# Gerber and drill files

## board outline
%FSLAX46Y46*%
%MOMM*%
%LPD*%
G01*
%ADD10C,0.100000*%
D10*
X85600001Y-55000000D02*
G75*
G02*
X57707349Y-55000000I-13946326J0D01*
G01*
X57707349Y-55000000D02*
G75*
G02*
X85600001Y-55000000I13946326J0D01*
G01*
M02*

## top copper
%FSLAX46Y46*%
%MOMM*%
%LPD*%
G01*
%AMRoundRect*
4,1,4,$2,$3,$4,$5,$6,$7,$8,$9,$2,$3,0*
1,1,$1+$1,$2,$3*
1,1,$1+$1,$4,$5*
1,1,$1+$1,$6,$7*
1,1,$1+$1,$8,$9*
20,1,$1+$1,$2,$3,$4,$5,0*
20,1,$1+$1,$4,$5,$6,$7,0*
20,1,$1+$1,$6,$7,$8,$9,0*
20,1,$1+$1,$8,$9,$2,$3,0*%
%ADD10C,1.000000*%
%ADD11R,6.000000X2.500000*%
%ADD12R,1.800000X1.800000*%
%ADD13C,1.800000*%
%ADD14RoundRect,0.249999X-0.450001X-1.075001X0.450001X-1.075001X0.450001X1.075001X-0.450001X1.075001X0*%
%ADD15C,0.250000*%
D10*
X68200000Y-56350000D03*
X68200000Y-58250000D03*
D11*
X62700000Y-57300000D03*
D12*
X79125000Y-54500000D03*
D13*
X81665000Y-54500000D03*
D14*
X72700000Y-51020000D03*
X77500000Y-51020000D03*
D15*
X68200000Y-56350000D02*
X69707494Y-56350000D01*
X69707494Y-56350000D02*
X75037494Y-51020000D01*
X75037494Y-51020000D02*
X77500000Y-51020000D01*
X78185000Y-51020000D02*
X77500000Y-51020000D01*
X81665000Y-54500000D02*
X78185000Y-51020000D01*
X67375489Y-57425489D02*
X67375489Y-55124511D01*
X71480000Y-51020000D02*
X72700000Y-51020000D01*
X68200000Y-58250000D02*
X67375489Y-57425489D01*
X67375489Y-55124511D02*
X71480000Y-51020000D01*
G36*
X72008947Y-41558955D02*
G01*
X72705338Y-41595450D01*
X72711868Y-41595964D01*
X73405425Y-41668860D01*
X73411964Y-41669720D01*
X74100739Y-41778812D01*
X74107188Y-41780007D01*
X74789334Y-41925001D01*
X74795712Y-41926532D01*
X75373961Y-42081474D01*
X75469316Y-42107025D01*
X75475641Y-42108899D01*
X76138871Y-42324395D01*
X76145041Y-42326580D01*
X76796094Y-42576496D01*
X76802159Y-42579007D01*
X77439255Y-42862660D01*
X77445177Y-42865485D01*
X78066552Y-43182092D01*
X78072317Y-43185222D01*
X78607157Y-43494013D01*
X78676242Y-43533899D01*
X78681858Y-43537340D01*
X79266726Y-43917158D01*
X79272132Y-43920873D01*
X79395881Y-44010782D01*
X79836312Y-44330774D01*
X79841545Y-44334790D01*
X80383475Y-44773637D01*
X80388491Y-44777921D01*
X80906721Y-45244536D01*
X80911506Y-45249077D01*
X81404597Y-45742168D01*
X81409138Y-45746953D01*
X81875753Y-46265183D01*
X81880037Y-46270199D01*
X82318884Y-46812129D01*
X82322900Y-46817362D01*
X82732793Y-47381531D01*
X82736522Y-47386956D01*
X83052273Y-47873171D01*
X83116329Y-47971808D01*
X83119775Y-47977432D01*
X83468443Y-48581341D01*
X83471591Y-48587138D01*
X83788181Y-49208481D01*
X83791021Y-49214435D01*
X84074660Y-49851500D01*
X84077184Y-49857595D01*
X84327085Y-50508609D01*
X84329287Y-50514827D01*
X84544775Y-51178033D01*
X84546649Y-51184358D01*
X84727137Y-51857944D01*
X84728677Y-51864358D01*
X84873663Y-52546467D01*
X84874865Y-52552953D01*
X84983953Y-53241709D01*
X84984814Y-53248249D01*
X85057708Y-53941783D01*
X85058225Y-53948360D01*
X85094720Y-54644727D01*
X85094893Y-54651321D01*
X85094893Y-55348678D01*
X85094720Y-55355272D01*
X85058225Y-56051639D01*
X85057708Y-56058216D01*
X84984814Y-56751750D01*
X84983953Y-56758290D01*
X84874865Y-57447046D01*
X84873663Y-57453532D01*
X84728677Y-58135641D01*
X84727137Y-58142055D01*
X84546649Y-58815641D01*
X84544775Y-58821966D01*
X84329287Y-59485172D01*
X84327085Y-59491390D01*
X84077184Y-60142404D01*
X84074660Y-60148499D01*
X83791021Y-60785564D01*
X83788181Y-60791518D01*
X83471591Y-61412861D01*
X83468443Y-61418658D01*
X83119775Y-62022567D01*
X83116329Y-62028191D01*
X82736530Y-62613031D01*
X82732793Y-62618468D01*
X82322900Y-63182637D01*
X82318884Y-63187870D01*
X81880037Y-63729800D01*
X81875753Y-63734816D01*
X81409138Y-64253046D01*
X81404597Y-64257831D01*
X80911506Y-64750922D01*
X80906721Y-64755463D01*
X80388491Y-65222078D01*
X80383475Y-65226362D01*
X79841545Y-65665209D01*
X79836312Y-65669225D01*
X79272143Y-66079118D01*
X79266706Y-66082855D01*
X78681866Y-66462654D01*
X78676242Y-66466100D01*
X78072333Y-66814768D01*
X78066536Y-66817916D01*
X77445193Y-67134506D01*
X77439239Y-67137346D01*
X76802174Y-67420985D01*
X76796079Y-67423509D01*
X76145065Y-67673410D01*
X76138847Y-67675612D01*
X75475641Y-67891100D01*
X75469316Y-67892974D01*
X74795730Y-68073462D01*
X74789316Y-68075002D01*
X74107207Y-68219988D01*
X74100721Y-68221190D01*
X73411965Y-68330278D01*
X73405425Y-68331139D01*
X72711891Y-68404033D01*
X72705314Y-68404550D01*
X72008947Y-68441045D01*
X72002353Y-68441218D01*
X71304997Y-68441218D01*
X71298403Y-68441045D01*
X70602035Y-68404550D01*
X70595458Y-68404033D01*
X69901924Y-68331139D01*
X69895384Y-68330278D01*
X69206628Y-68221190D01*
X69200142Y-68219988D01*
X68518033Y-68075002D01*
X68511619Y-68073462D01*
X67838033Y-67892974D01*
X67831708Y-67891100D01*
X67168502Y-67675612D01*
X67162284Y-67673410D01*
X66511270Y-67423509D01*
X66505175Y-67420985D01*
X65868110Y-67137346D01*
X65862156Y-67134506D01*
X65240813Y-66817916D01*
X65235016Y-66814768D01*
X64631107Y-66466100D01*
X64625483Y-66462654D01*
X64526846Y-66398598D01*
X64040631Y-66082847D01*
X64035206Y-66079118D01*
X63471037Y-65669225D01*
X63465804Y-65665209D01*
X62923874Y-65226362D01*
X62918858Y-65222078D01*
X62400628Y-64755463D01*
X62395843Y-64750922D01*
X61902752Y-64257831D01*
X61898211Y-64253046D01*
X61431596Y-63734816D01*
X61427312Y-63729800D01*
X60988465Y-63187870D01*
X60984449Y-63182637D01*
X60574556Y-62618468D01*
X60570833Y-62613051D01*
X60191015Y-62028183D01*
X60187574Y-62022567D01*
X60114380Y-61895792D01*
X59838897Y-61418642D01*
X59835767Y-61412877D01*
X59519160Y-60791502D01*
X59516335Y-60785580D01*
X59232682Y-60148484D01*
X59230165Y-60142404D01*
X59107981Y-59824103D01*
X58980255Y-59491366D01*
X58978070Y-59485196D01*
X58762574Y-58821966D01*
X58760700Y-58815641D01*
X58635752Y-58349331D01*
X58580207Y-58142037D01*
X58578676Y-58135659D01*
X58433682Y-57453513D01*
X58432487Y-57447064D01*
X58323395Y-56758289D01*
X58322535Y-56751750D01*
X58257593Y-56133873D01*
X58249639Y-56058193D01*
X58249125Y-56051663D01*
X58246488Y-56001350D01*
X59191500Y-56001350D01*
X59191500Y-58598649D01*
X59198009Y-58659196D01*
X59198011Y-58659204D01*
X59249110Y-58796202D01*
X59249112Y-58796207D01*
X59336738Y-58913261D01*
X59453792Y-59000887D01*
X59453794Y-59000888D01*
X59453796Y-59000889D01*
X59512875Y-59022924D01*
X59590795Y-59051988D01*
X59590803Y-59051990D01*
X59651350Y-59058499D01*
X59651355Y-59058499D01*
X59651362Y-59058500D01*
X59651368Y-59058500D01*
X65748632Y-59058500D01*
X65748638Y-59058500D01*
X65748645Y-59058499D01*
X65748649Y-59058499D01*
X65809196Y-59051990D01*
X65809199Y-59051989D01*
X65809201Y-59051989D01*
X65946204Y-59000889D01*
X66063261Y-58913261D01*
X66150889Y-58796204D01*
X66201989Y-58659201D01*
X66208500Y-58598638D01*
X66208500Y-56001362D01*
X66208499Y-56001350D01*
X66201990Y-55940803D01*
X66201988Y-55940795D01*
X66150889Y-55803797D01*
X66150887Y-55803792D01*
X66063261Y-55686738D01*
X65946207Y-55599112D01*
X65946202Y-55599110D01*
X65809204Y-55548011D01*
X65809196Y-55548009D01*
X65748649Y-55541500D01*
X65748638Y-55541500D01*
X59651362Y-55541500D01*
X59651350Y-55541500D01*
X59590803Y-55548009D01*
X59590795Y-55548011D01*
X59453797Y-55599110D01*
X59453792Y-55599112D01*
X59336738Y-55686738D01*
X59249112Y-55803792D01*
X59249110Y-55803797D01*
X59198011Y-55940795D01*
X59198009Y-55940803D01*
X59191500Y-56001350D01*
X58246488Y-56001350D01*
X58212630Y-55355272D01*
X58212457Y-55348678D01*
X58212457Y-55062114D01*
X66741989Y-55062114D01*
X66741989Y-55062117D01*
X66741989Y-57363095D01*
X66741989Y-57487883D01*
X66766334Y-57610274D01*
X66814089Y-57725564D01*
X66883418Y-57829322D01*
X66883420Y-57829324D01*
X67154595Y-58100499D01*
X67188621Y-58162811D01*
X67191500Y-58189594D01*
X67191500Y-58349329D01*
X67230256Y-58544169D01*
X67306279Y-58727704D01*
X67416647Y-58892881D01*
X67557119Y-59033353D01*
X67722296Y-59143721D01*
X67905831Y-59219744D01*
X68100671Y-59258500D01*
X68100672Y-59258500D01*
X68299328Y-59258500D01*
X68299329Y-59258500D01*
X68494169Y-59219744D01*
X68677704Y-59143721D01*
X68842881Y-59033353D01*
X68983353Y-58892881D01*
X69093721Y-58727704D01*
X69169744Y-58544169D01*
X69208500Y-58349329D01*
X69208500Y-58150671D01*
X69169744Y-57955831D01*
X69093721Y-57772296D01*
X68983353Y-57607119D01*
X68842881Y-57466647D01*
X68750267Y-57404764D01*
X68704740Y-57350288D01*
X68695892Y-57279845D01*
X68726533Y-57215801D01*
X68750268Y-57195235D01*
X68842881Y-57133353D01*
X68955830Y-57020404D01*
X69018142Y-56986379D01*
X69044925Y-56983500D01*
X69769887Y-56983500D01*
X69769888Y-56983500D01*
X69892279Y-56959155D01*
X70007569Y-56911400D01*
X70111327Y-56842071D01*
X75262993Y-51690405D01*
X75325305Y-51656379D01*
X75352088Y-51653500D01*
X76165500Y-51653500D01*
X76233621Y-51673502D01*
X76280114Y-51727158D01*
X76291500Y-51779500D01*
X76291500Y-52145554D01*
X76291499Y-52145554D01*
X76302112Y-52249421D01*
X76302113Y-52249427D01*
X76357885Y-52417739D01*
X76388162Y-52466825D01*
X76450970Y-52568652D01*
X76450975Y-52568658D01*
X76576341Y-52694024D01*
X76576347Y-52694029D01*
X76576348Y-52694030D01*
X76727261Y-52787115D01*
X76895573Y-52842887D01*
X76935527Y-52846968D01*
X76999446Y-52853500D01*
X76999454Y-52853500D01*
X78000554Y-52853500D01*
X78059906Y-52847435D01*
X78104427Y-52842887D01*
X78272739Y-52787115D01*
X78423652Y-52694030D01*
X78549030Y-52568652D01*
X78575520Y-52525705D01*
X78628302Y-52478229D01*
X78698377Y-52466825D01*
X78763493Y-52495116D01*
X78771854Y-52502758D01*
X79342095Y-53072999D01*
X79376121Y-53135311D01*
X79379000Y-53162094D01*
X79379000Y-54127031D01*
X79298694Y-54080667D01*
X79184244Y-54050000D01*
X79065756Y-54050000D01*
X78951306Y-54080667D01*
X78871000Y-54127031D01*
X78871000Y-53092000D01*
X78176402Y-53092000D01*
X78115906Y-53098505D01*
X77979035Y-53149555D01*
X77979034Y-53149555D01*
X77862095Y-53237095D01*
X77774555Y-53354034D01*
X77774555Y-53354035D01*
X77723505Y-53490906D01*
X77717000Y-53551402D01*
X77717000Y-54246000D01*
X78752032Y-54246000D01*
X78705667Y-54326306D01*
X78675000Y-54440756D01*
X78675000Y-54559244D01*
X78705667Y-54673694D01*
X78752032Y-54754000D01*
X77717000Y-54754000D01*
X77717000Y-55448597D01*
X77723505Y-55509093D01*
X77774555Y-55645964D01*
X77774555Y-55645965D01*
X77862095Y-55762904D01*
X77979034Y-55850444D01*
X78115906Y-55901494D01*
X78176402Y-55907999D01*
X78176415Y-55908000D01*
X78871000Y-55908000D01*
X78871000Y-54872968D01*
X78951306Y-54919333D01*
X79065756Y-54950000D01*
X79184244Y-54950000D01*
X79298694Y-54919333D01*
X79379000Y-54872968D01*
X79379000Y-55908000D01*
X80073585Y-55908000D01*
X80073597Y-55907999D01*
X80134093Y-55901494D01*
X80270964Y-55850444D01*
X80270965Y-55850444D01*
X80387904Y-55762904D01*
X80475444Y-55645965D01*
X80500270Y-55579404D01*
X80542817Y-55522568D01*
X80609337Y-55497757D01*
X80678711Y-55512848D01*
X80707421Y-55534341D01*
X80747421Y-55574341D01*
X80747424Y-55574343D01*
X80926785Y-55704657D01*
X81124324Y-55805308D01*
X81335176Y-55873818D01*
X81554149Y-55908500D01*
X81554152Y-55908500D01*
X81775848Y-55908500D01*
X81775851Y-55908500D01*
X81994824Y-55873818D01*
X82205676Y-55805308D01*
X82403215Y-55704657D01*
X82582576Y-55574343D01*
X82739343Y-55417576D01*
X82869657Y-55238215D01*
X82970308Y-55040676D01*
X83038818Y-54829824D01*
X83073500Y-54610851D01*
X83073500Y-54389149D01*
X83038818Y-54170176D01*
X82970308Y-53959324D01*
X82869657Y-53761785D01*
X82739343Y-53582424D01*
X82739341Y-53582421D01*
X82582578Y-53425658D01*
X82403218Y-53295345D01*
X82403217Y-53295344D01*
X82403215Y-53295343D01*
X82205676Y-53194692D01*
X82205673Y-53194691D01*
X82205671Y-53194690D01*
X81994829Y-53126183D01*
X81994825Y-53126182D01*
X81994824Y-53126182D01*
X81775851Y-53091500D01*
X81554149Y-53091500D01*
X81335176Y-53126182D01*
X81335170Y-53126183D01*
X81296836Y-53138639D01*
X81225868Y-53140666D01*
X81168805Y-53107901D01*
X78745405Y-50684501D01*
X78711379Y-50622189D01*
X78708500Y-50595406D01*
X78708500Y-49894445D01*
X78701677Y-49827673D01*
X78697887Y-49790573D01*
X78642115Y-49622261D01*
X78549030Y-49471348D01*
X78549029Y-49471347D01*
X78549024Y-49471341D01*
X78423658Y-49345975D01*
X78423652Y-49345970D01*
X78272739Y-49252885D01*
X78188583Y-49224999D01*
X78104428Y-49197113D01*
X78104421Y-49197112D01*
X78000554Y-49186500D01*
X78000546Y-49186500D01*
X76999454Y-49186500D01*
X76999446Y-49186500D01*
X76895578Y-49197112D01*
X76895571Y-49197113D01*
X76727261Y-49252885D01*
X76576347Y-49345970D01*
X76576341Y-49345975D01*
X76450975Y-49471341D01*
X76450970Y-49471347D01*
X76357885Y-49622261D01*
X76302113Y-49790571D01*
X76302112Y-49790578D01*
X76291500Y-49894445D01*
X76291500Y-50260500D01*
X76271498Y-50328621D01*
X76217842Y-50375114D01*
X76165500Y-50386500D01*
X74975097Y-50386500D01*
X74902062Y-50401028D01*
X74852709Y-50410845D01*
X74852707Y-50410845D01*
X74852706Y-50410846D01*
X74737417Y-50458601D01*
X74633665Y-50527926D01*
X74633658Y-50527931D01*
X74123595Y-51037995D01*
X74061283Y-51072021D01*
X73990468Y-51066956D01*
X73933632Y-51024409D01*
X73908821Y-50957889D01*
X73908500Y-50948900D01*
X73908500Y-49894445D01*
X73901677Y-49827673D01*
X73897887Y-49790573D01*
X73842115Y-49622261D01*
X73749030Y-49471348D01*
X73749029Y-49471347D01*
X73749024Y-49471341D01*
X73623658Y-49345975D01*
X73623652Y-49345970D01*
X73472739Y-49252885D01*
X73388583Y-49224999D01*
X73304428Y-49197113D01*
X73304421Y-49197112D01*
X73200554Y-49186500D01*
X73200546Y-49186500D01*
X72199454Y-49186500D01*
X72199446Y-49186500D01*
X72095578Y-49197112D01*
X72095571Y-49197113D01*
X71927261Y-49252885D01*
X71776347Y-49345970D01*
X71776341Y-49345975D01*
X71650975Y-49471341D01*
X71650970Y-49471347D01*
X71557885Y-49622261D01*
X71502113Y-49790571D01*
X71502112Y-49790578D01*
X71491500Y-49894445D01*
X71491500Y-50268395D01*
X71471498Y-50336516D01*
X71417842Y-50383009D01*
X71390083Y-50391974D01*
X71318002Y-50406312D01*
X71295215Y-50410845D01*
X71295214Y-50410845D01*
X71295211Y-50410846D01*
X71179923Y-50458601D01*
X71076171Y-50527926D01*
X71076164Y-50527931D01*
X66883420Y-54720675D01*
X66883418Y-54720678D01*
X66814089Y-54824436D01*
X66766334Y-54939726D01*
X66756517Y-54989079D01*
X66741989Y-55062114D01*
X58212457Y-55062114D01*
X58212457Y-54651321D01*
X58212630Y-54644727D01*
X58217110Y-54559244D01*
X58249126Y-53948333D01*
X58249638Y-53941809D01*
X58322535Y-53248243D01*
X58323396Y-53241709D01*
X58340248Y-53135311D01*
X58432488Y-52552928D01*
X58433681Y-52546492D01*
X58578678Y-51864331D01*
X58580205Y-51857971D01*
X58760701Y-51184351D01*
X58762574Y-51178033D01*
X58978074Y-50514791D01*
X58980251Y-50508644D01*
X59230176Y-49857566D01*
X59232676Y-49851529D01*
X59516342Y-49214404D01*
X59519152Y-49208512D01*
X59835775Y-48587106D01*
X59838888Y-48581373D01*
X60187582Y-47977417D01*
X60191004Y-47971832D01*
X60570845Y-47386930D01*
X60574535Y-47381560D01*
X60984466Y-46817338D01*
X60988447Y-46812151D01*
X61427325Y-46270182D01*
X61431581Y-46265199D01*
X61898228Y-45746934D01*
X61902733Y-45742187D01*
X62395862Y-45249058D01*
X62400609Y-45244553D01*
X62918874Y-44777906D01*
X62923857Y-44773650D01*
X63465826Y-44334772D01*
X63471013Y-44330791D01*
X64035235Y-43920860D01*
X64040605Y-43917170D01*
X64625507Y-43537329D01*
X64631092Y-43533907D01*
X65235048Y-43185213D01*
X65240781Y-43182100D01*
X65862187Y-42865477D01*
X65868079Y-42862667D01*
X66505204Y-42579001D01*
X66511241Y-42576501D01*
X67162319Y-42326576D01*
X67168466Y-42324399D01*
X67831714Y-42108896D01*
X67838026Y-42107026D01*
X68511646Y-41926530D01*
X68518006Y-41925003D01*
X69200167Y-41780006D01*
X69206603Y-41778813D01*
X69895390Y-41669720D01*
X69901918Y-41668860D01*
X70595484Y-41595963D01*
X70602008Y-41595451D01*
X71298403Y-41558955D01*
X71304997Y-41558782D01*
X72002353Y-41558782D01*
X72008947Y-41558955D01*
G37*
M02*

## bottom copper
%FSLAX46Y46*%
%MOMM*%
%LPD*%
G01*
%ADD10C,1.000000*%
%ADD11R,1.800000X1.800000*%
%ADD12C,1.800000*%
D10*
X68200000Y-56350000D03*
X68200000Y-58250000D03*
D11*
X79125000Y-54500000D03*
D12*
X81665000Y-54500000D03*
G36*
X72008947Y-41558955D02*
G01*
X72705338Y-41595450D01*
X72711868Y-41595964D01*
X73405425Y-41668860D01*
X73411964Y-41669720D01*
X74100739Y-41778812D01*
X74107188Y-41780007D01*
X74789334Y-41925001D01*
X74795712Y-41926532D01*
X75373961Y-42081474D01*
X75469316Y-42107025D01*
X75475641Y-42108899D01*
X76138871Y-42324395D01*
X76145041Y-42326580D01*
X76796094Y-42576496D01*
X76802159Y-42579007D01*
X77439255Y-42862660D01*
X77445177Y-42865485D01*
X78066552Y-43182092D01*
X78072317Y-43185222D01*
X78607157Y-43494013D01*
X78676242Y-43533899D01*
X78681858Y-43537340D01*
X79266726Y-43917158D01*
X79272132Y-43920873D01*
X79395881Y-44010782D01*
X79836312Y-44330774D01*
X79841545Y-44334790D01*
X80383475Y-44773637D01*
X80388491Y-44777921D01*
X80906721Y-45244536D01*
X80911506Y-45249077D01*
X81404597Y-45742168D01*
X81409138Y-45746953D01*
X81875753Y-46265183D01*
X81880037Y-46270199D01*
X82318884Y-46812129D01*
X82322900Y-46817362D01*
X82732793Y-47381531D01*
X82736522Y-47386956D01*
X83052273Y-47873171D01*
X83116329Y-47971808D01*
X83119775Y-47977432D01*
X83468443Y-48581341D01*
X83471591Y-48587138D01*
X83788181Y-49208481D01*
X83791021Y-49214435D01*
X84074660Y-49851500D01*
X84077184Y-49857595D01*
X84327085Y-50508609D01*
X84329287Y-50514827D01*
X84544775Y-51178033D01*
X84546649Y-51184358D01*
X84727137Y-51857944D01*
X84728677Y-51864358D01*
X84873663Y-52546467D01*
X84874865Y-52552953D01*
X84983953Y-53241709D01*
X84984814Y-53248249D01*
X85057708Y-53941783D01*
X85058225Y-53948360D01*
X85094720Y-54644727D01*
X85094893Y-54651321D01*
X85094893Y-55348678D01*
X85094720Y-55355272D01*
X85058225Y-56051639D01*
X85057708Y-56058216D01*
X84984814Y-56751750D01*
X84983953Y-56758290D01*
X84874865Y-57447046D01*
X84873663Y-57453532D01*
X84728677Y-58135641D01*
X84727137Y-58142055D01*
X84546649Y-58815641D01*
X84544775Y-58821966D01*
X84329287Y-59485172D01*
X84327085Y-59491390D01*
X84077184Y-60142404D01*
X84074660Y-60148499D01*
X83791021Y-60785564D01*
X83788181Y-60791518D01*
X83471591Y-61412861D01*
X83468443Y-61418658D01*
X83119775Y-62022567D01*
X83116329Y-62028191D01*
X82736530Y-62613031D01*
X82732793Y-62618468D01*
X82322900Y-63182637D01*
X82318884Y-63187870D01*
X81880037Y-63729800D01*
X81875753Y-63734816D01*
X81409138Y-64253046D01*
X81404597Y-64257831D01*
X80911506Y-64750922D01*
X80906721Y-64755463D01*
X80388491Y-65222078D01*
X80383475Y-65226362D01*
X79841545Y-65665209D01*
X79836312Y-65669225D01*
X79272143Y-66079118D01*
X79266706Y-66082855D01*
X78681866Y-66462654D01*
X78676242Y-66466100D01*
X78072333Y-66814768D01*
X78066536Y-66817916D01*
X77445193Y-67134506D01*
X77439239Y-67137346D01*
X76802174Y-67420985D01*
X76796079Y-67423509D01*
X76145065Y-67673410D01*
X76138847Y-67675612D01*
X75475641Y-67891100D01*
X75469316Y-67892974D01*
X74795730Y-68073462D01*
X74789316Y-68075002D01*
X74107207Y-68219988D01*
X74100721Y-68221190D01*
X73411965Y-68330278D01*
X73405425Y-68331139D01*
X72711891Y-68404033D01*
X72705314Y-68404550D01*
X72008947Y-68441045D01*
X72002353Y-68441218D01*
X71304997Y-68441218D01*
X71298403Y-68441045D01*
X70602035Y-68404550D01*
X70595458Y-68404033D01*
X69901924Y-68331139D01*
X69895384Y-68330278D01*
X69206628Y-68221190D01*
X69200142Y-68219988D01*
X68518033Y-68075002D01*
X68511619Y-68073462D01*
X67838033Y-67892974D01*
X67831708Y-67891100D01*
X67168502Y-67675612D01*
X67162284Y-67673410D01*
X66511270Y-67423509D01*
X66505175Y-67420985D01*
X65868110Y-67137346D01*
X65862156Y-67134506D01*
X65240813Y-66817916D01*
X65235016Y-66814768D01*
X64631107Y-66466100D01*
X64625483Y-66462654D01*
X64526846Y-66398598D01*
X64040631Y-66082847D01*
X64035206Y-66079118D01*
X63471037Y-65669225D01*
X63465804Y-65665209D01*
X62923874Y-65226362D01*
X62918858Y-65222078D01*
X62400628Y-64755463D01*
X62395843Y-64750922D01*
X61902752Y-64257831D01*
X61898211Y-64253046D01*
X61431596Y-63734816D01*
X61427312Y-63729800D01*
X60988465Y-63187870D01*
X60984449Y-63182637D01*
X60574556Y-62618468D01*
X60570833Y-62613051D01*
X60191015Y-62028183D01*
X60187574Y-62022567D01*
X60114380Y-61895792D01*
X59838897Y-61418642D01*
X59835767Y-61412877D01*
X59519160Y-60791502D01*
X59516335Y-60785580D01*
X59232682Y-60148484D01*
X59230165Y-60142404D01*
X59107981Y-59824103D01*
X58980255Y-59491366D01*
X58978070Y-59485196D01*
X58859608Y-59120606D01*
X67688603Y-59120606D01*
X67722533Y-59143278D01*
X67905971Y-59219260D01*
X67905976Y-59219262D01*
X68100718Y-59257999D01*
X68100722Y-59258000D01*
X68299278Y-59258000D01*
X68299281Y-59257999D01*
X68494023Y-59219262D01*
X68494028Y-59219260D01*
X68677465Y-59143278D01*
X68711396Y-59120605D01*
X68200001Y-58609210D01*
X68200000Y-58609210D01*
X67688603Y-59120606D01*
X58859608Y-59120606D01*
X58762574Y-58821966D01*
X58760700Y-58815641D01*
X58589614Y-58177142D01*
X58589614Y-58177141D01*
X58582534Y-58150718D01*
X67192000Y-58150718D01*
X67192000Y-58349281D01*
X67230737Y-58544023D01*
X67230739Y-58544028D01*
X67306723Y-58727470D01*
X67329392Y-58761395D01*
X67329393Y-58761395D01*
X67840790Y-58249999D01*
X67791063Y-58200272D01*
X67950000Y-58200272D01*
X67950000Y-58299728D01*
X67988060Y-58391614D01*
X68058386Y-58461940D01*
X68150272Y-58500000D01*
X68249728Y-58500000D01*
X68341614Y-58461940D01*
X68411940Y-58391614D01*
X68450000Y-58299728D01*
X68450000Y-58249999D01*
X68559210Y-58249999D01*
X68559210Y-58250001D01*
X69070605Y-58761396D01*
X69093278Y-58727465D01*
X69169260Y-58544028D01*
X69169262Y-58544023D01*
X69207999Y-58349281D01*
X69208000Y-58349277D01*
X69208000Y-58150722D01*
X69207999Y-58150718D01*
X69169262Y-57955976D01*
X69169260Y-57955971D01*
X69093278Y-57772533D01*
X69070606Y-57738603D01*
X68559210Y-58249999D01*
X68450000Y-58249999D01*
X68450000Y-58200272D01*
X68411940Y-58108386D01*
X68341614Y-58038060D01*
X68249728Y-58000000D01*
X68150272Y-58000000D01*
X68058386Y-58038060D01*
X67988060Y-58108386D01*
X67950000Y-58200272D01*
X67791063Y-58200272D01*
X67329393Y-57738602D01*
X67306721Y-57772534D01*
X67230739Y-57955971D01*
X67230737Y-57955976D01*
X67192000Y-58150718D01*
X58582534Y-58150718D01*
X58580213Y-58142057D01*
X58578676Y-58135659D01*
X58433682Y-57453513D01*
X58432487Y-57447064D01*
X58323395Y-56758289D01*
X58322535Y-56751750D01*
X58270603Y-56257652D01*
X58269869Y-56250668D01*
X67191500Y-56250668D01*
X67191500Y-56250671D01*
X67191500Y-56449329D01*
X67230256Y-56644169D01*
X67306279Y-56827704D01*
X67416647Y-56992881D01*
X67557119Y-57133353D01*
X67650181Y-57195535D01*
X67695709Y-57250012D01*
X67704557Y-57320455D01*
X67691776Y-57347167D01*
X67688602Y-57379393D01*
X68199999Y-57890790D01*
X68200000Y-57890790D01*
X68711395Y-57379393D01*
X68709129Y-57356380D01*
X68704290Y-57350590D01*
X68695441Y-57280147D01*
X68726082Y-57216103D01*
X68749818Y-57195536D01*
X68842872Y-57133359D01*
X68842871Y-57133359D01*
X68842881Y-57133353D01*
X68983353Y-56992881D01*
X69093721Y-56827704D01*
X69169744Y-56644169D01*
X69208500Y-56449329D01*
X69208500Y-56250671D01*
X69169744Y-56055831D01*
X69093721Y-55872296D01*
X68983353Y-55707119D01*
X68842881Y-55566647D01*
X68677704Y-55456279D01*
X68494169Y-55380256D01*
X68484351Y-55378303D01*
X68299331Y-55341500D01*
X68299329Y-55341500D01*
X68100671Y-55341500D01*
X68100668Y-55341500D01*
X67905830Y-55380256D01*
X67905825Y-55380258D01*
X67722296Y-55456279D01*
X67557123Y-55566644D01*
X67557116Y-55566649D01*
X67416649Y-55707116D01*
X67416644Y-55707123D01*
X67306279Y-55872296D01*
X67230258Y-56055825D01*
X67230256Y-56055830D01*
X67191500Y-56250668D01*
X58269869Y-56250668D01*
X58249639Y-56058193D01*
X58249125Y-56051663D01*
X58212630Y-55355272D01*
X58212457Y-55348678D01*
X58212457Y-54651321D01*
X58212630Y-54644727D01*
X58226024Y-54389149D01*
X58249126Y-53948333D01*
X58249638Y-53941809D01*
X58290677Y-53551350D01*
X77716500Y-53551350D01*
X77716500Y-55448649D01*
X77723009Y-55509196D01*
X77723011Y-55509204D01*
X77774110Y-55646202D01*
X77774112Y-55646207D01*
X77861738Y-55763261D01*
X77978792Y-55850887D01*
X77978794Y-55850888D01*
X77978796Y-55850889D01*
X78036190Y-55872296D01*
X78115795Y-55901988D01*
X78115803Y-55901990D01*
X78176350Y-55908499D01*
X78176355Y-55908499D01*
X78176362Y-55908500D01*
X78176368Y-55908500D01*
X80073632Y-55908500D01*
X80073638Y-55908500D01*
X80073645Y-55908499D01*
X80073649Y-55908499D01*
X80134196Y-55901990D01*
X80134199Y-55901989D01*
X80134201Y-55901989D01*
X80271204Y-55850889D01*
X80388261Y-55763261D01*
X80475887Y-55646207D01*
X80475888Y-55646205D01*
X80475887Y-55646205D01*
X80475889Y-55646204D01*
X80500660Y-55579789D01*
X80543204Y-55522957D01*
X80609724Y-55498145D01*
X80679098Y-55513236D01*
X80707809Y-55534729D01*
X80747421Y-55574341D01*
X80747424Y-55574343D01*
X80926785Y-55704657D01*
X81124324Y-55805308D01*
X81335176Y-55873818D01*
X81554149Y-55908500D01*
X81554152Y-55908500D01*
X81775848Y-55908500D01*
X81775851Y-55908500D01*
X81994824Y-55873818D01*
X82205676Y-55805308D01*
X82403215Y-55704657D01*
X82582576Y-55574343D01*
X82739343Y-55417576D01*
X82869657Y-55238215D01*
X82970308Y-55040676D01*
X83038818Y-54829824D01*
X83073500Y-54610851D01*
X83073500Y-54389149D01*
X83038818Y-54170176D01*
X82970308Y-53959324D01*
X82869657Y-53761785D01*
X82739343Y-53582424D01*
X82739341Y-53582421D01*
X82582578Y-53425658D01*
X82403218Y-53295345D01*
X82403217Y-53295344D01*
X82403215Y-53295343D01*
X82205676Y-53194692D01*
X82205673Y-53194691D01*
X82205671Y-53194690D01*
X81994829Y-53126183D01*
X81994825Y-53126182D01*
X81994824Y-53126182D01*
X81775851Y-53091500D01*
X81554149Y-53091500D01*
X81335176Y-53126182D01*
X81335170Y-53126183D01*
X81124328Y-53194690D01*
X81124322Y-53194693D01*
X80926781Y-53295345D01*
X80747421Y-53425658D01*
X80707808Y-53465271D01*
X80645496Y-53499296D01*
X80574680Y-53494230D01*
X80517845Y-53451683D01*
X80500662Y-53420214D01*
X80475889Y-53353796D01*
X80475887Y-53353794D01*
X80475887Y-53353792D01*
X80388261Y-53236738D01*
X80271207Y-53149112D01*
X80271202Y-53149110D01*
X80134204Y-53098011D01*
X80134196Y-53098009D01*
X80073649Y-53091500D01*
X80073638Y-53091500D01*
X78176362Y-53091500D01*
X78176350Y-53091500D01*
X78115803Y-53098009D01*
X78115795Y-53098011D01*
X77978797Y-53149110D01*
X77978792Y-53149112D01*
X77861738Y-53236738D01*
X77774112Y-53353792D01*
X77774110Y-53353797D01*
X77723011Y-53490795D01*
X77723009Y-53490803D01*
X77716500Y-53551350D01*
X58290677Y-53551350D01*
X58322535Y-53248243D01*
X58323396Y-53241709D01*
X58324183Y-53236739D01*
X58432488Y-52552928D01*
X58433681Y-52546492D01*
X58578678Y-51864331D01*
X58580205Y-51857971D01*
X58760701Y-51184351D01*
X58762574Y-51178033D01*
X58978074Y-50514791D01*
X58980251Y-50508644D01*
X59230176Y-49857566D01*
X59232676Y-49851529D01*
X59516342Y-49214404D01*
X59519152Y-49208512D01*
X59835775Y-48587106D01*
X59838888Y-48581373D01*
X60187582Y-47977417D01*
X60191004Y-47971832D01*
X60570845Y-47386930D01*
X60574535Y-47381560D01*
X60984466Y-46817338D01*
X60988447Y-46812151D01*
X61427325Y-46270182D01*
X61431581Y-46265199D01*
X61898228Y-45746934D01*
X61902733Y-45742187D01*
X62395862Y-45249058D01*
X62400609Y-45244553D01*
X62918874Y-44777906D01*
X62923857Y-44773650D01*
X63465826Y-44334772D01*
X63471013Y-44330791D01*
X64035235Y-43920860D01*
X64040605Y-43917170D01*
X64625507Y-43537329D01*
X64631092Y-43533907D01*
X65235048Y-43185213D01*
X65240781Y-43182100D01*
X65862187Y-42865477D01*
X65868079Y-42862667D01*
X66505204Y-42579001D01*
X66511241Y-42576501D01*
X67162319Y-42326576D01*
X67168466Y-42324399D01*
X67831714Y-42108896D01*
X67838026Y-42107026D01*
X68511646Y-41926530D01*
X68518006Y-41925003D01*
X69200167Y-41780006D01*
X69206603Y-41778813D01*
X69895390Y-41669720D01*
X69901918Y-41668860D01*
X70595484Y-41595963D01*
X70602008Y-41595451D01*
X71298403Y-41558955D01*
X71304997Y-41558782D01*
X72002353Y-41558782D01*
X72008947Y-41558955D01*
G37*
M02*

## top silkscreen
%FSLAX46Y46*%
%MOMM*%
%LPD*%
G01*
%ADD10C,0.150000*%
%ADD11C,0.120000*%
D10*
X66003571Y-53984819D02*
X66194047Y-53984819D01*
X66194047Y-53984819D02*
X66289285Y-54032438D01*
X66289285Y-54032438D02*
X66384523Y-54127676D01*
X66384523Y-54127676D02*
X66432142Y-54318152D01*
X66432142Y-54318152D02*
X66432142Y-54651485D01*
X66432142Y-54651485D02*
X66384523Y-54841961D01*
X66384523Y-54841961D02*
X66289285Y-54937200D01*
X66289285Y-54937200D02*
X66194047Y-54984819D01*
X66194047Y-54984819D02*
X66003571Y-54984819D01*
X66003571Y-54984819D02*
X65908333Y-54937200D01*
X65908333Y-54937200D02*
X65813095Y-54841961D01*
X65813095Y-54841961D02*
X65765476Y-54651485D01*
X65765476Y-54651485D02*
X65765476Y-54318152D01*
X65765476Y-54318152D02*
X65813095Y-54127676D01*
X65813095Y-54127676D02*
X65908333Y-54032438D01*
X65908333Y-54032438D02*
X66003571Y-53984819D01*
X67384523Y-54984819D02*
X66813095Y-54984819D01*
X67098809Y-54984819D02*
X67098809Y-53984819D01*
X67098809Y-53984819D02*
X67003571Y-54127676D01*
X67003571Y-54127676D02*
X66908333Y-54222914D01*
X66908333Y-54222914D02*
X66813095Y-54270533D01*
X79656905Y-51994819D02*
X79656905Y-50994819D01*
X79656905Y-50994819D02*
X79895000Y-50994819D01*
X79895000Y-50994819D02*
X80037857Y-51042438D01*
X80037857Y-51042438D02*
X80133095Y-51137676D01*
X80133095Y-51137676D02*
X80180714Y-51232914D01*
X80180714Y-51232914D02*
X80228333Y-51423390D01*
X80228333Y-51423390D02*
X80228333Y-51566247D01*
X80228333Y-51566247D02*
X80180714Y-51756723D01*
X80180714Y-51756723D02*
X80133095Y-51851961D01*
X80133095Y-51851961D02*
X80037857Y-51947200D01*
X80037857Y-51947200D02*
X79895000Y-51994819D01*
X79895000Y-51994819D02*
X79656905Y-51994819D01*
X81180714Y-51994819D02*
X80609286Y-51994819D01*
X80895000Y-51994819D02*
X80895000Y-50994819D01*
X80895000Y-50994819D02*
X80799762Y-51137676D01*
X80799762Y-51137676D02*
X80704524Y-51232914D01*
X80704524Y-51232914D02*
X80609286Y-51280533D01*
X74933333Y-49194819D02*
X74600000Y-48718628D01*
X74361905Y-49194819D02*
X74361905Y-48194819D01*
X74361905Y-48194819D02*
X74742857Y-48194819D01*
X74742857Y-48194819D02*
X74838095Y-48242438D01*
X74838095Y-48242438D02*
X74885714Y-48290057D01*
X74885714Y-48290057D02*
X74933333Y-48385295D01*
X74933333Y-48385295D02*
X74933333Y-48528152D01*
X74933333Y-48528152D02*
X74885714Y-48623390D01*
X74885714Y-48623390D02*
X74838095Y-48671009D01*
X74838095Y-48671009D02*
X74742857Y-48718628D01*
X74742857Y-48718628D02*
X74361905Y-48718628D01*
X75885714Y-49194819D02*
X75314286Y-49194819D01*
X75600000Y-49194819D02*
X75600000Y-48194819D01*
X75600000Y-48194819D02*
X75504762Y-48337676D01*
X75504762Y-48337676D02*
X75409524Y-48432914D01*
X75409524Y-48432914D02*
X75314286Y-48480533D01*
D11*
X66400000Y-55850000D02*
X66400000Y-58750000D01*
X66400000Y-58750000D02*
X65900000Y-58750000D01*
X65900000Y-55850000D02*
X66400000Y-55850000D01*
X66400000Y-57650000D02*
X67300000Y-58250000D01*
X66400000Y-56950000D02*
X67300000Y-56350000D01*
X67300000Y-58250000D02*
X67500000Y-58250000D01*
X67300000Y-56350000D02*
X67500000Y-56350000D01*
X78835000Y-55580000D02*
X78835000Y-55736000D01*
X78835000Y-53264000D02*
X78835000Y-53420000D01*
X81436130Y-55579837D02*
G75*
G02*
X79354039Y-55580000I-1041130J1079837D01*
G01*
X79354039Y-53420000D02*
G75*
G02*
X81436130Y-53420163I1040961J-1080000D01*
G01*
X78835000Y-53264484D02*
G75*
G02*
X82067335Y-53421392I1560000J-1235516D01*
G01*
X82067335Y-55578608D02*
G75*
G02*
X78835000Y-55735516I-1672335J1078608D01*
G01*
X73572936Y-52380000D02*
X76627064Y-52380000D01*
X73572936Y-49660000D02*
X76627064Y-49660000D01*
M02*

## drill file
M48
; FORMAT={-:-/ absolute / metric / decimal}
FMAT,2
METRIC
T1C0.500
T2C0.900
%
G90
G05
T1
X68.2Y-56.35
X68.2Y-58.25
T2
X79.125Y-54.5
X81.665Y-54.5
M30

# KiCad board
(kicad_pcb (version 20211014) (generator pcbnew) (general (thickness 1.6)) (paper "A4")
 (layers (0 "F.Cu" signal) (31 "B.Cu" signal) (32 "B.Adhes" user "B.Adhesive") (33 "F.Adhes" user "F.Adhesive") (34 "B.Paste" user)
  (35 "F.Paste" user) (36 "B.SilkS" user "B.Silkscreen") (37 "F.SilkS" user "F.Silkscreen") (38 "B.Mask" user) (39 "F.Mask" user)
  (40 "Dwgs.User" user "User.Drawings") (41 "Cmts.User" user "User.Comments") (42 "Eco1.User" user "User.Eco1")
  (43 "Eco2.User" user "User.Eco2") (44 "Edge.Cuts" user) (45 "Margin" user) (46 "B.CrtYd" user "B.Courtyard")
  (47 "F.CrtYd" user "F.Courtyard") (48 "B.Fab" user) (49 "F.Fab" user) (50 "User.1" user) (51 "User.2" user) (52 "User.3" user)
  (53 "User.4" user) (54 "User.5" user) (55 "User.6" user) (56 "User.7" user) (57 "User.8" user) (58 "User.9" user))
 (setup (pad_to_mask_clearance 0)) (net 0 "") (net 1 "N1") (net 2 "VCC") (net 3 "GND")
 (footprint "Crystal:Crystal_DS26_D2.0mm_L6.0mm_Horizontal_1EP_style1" (layer "F.Cu") (at 68.2 56.35 -90)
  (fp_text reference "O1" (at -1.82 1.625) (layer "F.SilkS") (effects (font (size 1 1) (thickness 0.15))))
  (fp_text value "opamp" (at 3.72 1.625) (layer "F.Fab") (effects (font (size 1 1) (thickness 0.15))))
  (fp_line (start -0.5 1.8) (end 2.4 1.8) (layer "F.SilkS") (width 0.12))
  (fp_line (start 2.4 1.8) (end 2.4 2.3) (layer "F.SilkS") (width 0.12))
  (fp_line (start -0.5 2.3) (end -0.5 1.8) (layer "F.SilkS") (width 0.12))
  (fp_line (start 1.3 1.8) (end 1.9 0.9) (layer "F.SilkS") (width 0.12))
  (fp_line (start 0.6 1.8) (end 0 0.9) (layer "F.SilkS") (width 0.12))
  (fp_line (start 1.9 0.9) (end 1.9 0.7) (layer "F.SilkS") (width 0.12))
  (fp_line (start 0 0.9) (end 0 0.7) (layer "F.SilkS") (width 0.12))
  (pad "1" thru_hole circle (at 0 0 270) (size 1 1) (drill 0.5) (layers *.Cu *.Mask) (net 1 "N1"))
  (pad "2" thru_hole circle (at 1.9 0 270) (size 1 1) (drill 0.5) (layers *.Cu *.Mask) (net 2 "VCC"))
  (pad "3" smd rect (at 0.95 5.5 270) (size 2.5 6) (layers "F.Cu" "F.Paste" "F.Mask")))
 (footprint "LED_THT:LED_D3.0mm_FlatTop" (layer "F.Cu") (at 79.125 54.5)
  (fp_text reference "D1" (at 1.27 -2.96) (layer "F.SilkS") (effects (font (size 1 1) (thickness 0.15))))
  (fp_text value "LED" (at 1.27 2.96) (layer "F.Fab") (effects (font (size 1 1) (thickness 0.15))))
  (fp_line (start -0.29 1.08) (end -0.29 1.236) (layer "F.SilkS") (width 0.12))
  (fp_line (start -0.29 -1.236) (end -0.29 -1.08) (layer "F.SilkS") (width 0.12))
  (fp_arc (start 2.31113 1.079837) (mid 1.270117 1.5) (end 0.229039 1.08) (layer "F.SilkS") (width 0.12))
  (fp_arc (start 0.229039 -1.08) (mid 1.270117 -1.5) (end 2.31113 -1.079837) (layer "F.SilkS") (width 0.12))
  (fp_arc (start -0.29 -1.235516) (mid 1.366487 -1.987659) (end 2.942335 -1.078608) (layer "F.SilkS") (width 0.12))
  (fp_arc (start 2.942335 1.078608) (mid 1.366487 1.987659) (end -0.29 1.235516) (layer "F.SilkS") (width 0.12))
  (pad "1" thru_hole rect (at 0 0) (size 1.8 1.8) (drill 0.9) (layers *.Cu *.Mask) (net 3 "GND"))
  (pad "2" thru_hole circle (at 2.54 0) (size 1.8 1.8) (drill 0.9) (layers *.Cu *.Mask) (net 1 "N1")))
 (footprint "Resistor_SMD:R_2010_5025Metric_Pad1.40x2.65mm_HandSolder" (layer "F.Cu") (at 75.1 51.02)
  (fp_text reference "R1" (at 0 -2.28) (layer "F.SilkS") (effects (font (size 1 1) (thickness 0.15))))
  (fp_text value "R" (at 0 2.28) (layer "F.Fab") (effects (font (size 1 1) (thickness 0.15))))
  (fp_line (start -1.527064 1.36) (end 1.527064 1.36) (layer "F.SilkS") (width 0.12))
  (fp_line (start -1.527064 -1.36) (end 1.527064 -1.36) (layer "F.SilkS") (width 0.12))
  (pad "1" smd roundrect (at -2.4 0) (size 1.4 2.65) (layers "F.Cu" "F.Paste" "F.Mask") (roundrect_rratio 0.178571) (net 2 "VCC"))
  (pad "2" smd roundrect (at 2.4 0) (size 1.4 2.65) (layers "F.Cu" "F.Paste" "F.Mask") (roundrect_rratio 0.178571) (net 1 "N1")))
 (gr_circle (center 71.653675 55) (end 84.553675 60.3) (layer "Edge.Cuts") (width 0.1) (fill none))
 (segment (start 68.2 56.35) (end 69.707494 56.35) (width 0.25) (layer "F.Cu") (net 1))
 (segment (start 69.707494 56.35) (end 75.037494 51.02) (width 0.25) (layer "F.Cu") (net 1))
 (segment (start 75.037494 51.02) (end 77.5 51.02) (width 0.25) (layer "F.Cu") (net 1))
 (segment (start 78.185 51.02) (end 77.5 51.02) (width 0.25) (layer "F.Cu") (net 1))
 (segment (start 81.665 54.5) (end 78.185 51.02) (width 0.25) (layer "F.Cu") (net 1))
 (segment (start 67.375489 57.425489) (end 67.375489 55.124511) (width 0.25) (layer "F.Cu") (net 2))
 (segment (start 71.48 51.02) (end 72.7 51.02) (width 0.25) (layer "F.Cu") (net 2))
 (segment (start 68.2 58.25) (end 67.375489 57.425489) (width 0.25) (layer "F.Cu") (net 2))
 (segment (start 67.375489 55.124511) (end 71.48 51.02) (width 0.25) (layer "F.Cu") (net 2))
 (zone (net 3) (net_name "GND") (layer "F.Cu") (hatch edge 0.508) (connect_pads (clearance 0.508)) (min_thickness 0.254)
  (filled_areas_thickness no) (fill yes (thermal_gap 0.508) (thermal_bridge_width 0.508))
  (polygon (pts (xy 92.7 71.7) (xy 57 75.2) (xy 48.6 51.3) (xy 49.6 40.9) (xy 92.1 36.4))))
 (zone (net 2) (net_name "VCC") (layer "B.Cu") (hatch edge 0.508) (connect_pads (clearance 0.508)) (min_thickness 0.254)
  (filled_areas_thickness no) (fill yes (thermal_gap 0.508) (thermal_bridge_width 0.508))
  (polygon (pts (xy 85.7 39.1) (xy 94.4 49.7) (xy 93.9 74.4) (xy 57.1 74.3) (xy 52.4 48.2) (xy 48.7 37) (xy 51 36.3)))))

